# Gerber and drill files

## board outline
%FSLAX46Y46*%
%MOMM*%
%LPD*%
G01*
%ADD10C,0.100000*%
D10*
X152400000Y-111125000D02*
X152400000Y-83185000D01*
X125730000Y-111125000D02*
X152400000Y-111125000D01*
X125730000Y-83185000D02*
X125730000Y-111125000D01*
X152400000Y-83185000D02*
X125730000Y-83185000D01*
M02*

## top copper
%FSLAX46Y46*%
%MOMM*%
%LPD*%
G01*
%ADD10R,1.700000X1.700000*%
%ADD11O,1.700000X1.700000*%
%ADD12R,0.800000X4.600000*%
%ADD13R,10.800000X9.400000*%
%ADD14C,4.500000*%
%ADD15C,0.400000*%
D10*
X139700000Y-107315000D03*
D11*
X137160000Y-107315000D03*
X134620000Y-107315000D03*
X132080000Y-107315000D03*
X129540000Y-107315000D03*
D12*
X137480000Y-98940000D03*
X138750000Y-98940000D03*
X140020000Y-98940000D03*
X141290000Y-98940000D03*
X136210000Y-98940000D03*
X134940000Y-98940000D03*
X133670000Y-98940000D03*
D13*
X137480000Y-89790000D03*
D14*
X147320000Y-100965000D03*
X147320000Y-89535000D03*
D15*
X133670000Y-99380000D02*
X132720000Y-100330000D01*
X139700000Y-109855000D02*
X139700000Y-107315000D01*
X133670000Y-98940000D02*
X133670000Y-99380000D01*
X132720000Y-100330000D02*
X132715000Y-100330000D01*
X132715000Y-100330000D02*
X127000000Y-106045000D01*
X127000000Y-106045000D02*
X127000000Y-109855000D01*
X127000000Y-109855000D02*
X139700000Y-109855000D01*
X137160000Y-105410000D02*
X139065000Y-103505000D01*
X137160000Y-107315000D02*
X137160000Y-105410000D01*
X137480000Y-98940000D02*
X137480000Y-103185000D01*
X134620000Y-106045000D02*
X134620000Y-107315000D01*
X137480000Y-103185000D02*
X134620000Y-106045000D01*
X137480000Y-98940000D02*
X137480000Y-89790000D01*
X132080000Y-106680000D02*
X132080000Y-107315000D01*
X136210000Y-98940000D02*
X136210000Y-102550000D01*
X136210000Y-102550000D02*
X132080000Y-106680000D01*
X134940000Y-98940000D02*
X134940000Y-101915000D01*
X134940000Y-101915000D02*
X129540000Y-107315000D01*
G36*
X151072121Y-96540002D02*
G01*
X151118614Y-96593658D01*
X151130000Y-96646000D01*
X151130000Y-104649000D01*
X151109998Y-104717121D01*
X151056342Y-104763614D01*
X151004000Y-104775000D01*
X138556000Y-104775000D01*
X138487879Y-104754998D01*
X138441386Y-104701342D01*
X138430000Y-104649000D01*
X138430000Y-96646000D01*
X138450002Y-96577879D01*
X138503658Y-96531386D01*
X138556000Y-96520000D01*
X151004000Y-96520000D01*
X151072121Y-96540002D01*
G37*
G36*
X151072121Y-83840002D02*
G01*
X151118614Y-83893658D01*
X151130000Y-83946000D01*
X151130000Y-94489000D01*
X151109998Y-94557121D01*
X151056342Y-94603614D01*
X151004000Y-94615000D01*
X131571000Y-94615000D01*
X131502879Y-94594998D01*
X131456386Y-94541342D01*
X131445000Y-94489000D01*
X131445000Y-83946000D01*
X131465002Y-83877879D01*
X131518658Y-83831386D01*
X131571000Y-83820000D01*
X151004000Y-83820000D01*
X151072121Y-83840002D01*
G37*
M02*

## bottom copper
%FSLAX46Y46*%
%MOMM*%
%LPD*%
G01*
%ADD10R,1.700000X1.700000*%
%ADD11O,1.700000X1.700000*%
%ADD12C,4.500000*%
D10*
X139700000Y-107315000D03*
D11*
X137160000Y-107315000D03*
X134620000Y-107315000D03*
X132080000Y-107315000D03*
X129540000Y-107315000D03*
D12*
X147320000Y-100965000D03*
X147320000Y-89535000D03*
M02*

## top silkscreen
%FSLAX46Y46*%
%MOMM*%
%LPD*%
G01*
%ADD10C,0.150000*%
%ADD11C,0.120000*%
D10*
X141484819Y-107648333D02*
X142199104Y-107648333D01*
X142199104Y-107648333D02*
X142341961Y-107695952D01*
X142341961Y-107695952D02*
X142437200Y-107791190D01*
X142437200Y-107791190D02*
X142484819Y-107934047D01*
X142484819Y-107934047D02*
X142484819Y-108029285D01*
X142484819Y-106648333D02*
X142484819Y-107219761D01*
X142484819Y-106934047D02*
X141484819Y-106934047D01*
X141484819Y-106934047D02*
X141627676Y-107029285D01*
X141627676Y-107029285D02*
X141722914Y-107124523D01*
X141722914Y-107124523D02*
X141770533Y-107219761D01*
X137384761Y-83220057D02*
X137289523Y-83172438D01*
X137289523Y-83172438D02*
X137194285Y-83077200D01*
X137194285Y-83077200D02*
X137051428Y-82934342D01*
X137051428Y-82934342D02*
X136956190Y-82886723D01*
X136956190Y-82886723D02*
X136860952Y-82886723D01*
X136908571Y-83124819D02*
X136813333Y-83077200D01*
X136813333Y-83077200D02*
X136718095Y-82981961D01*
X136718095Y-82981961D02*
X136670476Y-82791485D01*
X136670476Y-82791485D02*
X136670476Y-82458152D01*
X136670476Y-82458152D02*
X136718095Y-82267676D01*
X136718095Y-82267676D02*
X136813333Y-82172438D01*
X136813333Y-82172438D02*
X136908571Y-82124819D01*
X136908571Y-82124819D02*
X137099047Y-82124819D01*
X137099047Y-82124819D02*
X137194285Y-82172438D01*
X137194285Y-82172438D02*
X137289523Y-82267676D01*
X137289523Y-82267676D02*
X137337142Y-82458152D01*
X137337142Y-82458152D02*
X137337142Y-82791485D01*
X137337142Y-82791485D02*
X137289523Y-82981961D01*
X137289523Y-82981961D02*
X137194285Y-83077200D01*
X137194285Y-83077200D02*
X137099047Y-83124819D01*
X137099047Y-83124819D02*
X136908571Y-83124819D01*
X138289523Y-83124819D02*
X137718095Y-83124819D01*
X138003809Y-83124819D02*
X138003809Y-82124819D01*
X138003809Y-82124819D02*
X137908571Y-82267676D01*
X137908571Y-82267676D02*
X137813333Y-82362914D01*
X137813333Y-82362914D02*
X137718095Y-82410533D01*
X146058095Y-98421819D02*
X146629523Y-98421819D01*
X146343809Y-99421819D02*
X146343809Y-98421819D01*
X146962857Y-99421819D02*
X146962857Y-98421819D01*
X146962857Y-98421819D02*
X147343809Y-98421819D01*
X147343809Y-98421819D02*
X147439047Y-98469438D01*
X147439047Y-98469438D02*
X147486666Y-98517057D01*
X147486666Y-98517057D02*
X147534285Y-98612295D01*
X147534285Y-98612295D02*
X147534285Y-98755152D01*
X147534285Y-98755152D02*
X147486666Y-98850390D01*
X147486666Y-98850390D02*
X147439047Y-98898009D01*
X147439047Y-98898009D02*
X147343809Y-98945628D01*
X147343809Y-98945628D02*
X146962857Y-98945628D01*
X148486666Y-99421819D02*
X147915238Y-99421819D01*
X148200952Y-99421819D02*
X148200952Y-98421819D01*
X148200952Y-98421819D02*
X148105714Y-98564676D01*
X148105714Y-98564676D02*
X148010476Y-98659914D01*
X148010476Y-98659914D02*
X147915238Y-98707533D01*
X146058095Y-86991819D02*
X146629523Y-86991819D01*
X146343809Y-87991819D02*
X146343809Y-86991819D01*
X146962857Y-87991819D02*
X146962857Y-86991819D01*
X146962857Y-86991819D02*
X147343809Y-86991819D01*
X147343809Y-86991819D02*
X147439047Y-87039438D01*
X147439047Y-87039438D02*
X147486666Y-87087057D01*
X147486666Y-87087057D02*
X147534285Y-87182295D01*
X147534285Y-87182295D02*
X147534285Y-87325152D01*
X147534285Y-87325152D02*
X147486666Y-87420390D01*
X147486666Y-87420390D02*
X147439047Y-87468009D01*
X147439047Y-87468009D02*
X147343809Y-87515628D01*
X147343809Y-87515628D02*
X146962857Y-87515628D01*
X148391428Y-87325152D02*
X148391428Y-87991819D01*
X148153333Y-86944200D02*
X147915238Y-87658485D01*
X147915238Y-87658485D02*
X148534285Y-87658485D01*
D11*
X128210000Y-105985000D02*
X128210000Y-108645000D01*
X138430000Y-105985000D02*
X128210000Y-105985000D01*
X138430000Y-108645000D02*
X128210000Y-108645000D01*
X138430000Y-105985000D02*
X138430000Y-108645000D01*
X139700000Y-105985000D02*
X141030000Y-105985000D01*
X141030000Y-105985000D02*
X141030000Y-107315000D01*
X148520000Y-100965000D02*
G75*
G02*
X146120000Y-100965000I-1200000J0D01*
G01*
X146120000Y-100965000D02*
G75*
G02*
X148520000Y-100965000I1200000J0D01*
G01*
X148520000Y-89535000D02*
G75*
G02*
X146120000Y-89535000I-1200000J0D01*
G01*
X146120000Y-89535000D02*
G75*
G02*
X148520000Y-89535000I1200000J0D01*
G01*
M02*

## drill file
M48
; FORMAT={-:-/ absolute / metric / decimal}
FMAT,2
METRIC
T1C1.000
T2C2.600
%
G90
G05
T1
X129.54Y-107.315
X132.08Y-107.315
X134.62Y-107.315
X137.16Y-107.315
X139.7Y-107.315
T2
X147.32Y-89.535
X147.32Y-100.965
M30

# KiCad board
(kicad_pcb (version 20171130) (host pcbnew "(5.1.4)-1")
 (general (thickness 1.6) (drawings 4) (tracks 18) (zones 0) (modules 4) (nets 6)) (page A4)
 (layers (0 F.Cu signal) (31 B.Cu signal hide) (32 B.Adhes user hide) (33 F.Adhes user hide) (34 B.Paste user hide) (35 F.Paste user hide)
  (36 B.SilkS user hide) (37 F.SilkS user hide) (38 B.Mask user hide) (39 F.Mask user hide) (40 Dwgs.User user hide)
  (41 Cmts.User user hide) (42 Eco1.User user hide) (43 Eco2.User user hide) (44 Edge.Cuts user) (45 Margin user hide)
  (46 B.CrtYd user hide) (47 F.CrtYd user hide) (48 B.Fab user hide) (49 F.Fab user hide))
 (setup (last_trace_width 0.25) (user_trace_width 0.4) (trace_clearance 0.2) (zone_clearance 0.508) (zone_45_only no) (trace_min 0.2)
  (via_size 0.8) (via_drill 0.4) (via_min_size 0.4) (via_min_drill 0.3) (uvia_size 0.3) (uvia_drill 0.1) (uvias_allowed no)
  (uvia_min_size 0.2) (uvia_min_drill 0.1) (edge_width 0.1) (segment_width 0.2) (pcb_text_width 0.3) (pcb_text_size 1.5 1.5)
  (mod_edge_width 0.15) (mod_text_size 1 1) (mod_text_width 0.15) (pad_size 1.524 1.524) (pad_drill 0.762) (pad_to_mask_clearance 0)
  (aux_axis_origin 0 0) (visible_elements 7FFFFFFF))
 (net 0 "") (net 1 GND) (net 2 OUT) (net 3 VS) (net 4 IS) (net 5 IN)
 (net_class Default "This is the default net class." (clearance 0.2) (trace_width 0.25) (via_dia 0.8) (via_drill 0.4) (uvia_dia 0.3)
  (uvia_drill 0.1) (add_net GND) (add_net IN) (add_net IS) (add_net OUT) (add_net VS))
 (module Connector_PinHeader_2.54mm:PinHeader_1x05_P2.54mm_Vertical (layer F.Cu) (at 139.7 107.315 270)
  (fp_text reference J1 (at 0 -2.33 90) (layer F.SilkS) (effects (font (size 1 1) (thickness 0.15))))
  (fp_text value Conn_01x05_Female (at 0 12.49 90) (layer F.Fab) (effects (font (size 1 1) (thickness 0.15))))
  (fp_line (start -1.33 11.49) (end 1.33 11.49) (layer F.SilkS) (width 0.12))
  (fp_line (start -1.33 1.27) (end -1.33 11.49) (layer F.SilkS) (width 0.12))
  (fp_line (start 1.33 1.27) (end 1.33 11.49) (layer F.SilkS) (width 0.12))
  (fp_line (start -1.33 1.27) (end 1.33 1.27) (layer F.SilkS) (width 0.12))
  (fp_line (start -1.33 0) (end -1.33 -1.33) (layer F.SilkS) (width 0.12))
  (fp_line (start -1.33 -1.33) (end 0 -1.33) (layer F.SilkS) (width 0.12))
  (pad 1 thru_hole rect (at 0 0 270) (size 1.7 1.7) (drill 1) (layers *.Cu *.Mask) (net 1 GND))
  (pad 2 thru_hole oval (at 0 2.54 270) (size 1.7 1.7) (drill 1) (layers *.Cu *.Mask) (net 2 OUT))
  (pad 3 thru_hole oval (at 0 5.08 270) (size 1.7 1.7) (drill 1) (layers *.Cu *.Mask) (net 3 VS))
  (pad 4 thru_hole oval (at 0 7.62 270) (size 1.7 1.7) (drill 1) (layers *.Cu *.Mask) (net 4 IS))
  (pad 5 thru_hole oval (at 0 10.16 270) (size 1.7 1.7) (drill 1) (layers *.Cu *.Mask) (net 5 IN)))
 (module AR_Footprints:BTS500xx (layer F.Cu) (at 137.48 96.64)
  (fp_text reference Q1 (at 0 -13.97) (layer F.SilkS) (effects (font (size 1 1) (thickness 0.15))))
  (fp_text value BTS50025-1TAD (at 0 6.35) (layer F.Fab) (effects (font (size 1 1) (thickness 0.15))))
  (pad 4 smd rect (at 0 2.3) (size 0.8 4.6) (layers F.Cu F.Paste F.Mask) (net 3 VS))
  (pad 5 smd rect (at 1.27 2.3) (size 0.8 4.6) (layers F.Cu F.Paste F.Mask) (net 2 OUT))
  (pad 6 smd rect (at 2.54 2.3) (size 0.8 4.6) (layers F.Cu F.Paste F.Mask) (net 2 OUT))
  (pad 7 smd rect (at 3.81 2.3) (size 0.8 4.6) (layers F.Cu F.Paste F.Mask) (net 2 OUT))
  (pad 3 smd rect (at -1.27 2.3) (size 0.8 4.6) (layers F.Cu F.Paste F.Mask) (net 4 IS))
  (pad 2 smd rect (at -2.54 2.3) (size 0.8 4.6) (layers F.Cu F.Paste F.Mask) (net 5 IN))
  (pad 1 smd rect (at -3.81 2.3) (size 0.8 4.6) (layers F.Cu F.Paste F.Mask) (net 1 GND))
  (pad 8 smd rect (at 0 -6.85) (size 10.8 9.4) (layers F.Cu F.Paste F.Mask) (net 3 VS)))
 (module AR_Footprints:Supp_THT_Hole (layer F.Cu) (at 147.32 100.965)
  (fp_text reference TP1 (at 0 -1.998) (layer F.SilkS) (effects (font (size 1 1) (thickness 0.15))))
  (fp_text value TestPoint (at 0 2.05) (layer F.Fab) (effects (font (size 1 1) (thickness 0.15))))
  (fp_circle (center 0 0) (end 0 1.2) (layer F.SilkS) (width 0.12))
  (pad 1 thru_hole circle (at 0 0) (size 4.5 4.5) (drill 2.6) (layers *.Cu *.Mask) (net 2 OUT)))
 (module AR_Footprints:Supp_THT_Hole (layer F.Cu) (at 147.32 89.535)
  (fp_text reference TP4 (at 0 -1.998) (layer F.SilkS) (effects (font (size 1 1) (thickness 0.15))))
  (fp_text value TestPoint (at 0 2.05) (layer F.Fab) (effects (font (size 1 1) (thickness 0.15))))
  (fp_circle (center 0 0) (end 0 1.2) (layer F.SilkS) (width 0.12))
  (pad 1 thru_hole circle (at 0 0) (size 4.5 4.5) (drill 2.6) (layers *.Cu *.Mask) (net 3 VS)))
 (gr_line (start 152.4 111.125) (end 152.4 83.185) (layer Edge.Cuts) (width 0.1))
 (gr_line (start 125.73 111.125) (end 152.4 111.125) (layer Edge.Cuts) (width 0.1))
 (gr_line (start 125.73 83.185) (end 125.73 111.125) (layer Edge.Cuts) (width 0.1))
 (gr_line (start 152.4 83.185) (end 125.73 83.185) (layer Edge.Cuts) (width 0.1))
 (segment (start 133.67 99.38) (end 132.72 100.33) (width 0.4) (layer F.Cu) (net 1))
 (segment (start 139.7 109.855) (end 139.7 107.315) (width 0.4) (layer F.Cu) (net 1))
 (segment (start 133.67 98.94) (end 133.67 99.38) (width 0.4) (layer F.Cu) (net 1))
 (segment (start 132.72 100.33) (end 132.715 100.33) (width 0.4) (layer F.Cu) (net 1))
 (segment (start 132.715 100.33) (end 127 106.045) (width 0.4) (layer F.Cu) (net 1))
 (segment (start 127 106.045) (end 127 109.855) (width 0.4) (layer F.Cu) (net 1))
 (segment (start 127 109.855) (end 139.7 109.855) (width 0.4) (layer F.Cu) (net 1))
 (segment (start 137.16 105.41) (end 139.065 103.505) (width 0.4) (layer F.Cu) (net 2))
 (segment (start 137.16 107.315) (end 137.16 105.41) (width 0.4) (layer F.Cu) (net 2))
 (segment (start 137.48 98.94) (end 137.48 103.185) (width 0.4) (layer F.Cu) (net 3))
 (segment (start 134.62 106.045) (end 134.62 107.315) (width 0.4) (layer F.Cu) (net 3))
 (segment (start 137.48 103.185) (end 134.62 106.045) (width 0.4) (layer F.Cu) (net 3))
 (segment (start 137.48 98.94) (end 137.48 89.79) (width 0.4) (layer F.Cu) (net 3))
 (segment (start 132.08 106.68) (end 132.08 107.315) (width 0.4) (layer F.Cu) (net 4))
 (segment (start 136.21 98.94) (end 136.21 102.55) (width 0.4) (layer F.Cu) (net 4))
 (segment (start 136.21 102.55) (end 132.08 106.68) (width 0.4) (layer F.Cu) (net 4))
 (segment (start 134.94 98.94) (end 134.94 101.915) (width 0.4) (layer F.Cu) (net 5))
 (segment (start 134.94 101.915) (end 129.54 107.315) (width 0.4) (layer F.Cu) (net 5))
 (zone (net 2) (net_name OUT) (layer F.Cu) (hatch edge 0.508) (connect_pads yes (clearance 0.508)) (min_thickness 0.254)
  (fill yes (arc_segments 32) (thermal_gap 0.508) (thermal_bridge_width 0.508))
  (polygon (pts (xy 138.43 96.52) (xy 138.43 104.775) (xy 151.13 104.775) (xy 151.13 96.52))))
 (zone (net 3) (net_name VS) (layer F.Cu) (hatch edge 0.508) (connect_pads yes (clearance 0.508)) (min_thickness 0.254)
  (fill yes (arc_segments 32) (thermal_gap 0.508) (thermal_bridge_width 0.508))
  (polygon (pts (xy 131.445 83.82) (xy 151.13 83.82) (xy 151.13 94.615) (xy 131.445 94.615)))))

